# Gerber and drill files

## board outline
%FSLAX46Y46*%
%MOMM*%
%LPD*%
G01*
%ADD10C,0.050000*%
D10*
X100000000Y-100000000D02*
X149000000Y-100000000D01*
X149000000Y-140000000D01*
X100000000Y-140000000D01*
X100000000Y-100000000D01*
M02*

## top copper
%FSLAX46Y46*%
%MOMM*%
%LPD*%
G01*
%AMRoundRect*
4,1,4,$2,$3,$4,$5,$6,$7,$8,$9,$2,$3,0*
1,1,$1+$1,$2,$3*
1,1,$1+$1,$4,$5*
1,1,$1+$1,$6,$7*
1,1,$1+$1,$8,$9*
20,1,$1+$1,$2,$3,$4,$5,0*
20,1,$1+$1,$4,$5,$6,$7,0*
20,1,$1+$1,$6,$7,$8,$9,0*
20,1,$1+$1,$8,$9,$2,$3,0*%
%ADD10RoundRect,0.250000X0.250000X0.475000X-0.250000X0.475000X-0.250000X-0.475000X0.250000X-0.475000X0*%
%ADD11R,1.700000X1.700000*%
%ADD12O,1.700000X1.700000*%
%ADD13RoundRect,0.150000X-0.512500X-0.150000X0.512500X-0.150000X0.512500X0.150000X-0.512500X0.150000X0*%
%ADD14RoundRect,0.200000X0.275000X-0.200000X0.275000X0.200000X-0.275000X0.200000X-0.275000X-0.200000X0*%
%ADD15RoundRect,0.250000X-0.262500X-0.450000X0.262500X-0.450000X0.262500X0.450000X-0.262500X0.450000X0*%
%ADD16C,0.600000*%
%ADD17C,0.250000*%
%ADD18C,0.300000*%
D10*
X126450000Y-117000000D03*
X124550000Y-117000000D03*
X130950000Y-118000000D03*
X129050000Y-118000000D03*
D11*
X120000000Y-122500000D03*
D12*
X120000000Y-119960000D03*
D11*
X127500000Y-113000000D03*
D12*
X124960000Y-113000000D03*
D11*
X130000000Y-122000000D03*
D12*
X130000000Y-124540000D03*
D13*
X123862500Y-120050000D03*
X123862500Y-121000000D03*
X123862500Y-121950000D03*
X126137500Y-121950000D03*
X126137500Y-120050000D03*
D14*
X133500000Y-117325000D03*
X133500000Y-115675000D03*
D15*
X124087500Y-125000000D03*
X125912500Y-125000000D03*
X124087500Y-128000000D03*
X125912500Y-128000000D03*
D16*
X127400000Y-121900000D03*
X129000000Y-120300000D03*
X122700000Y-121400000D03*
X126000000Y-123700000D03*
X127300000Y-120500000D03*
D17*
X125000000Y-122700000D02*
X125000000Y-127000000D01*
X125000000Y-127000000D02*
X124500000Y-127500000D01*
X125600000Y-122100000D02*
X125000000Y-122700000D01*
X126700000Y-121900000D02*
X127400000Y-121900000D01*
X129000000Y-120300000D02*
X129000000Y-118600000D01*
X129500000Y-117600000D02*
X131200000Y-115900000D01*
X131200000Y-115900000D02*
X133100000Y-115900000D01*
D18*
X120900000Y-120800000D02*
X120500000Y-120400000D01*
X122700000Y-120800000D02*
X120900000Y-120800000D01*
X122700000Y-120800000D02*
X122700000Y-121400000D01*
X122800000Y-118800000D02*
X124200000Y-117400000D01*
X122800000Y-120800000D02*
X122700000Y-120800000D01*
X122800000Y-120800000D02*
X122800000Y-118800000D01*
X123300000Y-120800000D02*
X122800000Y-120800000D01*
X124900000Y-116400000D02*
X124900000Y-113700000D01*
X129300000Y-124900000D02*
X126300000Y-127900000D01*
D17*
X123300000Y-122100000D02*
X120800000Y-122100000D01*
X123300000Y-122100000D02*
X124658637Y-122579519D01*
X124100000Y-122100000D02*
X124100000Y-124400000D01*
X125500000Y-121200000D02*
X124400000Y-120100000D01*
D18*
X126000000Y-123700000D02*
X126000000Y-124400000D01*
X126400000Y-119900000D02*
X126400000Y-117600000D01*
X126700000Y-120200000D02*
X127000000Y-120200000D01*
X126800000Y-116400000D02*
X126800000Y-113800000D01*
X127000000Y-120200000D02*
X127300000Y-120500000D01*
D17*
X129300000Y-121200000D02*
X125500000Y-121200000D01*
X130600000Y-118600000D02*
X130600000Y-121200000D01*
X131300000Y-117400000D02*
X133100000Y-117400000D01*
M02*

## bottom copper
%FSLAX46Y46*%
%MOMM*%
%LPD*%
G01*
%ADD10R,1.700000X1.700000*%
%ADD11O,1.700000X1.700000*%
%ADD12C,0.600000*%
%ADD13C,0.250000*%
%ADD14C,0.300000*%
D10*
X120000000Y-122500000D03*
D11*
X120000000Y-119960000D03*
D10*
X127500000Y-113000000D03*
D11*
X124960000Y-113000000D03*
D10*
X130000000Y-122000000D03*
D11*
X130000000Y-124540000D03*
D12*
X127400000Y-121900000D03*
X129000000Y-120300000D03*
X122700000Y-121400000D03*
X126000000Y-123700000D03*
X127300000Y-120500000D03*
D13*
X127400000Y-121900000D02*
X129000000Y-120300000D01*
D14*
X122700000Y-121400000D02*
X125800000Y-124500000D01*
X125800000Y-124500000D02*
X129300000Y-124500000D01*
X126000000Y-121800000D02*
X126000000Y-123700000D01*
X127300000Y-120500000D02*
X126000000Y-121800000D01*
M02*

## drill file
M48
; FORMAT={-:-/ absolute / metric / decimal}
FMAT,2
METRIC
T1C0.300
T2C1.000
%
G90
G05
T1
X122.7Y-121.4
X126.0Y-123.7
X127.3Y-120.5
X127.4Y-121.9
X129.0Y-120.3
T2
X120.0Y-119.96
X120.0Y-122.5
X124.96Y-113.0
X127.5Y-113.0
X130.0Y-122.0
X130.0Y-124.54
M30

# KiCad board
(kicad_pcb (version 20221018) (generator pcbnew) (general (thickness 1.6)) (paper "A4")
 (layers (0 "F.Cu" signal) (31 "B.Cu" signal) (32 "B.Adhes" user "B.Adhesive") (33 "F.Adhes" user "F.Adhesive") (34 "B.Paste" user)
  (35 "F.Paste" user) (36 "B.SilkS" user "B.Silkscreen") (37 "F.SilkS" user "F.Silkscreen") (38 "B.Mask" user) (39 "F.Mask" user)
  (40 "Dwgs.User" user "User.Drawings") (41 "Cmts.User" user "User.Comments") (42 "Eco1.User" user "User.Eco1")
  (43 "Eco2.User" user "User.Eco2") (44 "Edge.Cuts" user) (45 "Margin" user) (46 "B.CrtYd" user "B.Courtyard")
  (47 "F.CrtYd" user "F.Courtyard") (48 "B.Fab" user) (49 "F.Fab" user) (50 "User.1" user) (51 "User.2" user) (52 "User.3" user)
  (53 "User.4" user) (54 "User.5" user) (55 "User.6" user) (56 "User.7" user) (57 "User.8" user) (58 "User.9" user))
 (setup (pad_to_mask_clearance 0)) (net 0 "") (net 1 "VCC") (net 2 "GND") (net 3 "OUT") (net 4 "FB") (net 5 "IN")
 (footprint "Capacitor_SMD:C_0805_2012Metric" (layer "F.Cu") (at 125.5 117 180)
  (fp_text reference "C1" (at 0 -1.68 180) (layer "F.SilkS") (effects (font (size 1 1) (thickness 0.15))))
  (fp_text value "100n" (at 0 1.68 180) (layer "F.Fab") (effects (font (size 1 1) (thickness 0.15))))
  (pad "1" smd roundrect (at -0.95 0 180) (size 1 1.45) (layers "F.Cu" "F.Paste" "F.Mask") (roundrect_rratio 0.25) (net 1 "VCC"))
  (pad "2" smd roundrect (at 0.95 0 180) (size 1 1.45) (layers "F.Cu" "F.Paste" "F.Mask") (roundrect_rratio 0.25) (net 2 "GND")))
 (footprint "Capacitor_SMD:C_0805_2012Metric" (layer "F.Cu") (at 130 118 180)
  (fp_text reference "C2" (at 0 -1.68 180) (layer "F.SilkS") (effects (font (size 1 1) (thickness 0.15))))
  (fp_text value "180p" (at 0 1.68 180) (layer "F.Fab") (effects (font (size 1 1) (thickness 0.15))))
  (pad "1" smd roundrect (at -0.95 0 180) (size 1 1.45) (layers "F.Cu" "F.Paste" "F.Mask") (roundrect_rratio 0.25) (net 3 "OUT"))
  (pad "2" smd roundrect (at 0.95 0 180) (size 1 1.45) (layers "F.Cu" "F.Paste" "F.Mask") (roundrect_rratio 0.25) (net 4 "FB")))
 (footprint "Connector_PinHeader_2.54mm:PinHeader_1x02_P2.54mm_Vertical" (layer "F.Cu") (at 120 122.5 180)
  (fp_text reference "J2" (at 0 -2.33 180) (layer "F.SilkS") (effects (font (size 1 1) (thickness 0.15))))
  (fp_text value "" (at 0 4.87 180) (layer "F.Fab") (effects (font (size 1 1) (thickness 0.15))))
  (pad "1" thru_hole rect (at 0 0 180) (size 1.7 1.7) (drill 1) (layers "*.Cu" "*.Mask") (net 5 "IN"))
  (pad "2" thru_hole oval (at 0 2.54 180) (size 1.7 1.7) (drill 1) (layers "*.Cu" "*.Mask") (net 2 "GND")))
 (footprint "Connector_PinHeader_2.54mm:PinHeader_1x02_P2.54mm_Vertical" (layer "F.Cu") (at 127.5 113 -90)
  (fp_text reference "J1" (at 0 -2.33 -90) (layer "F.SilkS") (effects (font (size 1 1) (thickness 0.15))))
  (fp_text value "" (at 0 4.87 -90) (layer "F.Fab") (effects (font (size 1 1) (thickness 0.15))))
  (pad "1" thru_hole rect (at 0 0 270) (size 1.7 1.7) (drill 1) (layers "*.Cu" "*.Mask") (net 1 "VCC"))
  (pad "2" thru_hole oval (at 0 2.54 270) (size 1.7 1.7) (drill 1) (layers "*.Cu" "*.Mask") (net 2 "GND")))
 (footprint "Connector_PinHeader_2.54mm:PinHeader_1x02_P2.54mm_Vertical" (layer "F.Cu") (at 130 122)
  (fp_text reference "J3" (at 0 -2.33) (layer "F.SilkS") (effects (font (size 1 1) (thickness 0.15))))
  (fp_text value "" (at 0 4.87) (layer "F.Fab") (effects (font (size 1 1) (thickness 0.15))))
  (pad "1" thru_hole rect (at 0 0) (size 1.7 1.7) (drill 1) (layers "*.Cu" "*.Mask") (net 3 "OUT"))
  (pad "2" thru_hole oval (at 0 2.54) (size 1.7 1.7) (drill 1) (layers "*.Cu" "*.Mask") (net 2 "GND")))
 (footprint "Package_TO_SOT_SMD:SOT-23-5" (layer "F.Cu") (at 125 121)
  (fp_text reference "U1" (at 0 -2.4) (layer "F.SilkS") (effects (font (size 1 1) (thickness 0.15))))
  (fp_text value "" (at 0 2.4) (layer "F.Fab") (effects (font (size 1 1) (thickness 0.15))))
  (pad "1" smd roundrect (at -1.1375 -0.95) (size 1.325 0.6) (layers "F.Cu" "F.Paste" "F.Mask") (roundrect_rratio 0.25) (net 3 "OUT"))
  (pad "2" smd roundrect (at -1.1375 0) (size 1.325 0.6) (layers "F.Cu" "F.Paste" "F.Mask") (roundrect_rratio 0.25) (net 2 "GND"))
  (pad "3" smd roundrect (at -1.1375 0.95) (size 1.325 0.6) (layers "F.Cu" "F.Paste" "F.Mask") (roundrect_rratio 0.25) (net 5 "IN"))
  (pad "4" smd roundrect (at 1.1375 0.95) (size 1.325 0.6) (layers "F.Cu" "F.Paste" "F.Mask") (roundrect_rratio 0.25) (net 4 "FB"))
  (pad "5" smd roundrect (at 1.1375 -0.95) (size 1.325 0.6) (layers "F.Cu" "F.Paste" "F.Mask") (roundrect_rratio 0.25) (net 1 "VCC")))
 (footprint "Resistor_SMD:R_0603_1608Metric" (layer "F.Cu") (at 133.5 116.5 90)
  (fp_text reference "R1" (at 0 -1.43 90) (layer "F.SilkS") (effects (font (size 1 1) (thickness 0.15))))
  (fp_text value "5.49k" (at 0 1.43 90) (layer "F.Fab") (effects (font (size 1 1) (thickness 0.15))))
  (pad "1" smd roundrect (at -0.825 0 90) (size 0.8 0.95) (layers "F.Cu" "F.Paste" "F.Mask") (roundrect_rratio 0.25) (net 3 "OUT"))
  (pad "2" smd roundrect (at 0.825 0 90) (size 0.8 0.95) (layers "F.Cu" "F.Paste" "F.Mask") (roundrect_rratio 0.25) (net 4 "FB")))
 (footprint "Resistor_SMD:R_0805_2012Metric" (layer "F.Cu") (at 125 125)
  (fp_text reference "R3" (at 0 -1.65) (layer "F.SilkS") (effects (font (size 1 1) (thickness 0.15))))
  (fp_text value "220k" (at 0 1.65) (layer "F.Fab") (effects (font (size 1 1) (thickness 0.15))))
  (pad "1" smd roundrect (at -0.9125 0) (size 1.025 1.4) (layers "F.Cu" "F.Paste" "F.Mask") (roundrect_rratio 0.243902) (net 5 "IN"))
  (pad "2" smd roundrect (at 0.9125 0) (size 1.025 1.4) (layers "F.Cu" "F.Paste" "F.Mask") (roundrect_rratio 0.243902) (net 1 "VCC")))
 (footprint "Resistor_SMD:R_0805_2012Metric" (layer "F.Cu") (at 125 128)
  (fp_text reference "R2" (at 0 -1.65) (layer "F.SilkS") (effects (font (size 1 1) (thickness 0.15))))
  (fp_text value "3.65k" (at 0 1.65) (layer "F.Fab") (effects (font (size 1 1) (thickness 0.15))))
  (pad "1" smd roundrect (at -0.9125 0) (size 1.025 1.4) (layers "F.Cu" "F.Paste" "F.Mask") (roundrect_rratio 0.243902) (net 4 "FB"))
  (pad "2" smd roundrect (at 0.9125 0) (size 1.025 1.4) (layers "F.Cu" "F.Paste" "F.Mask") (roundrect_rratio 0.243902) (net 2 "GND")))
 (gr_rect (start 100 100) (end 149 140) (stroke (width 0.05) (type default)) (fill none) (layer "Edge.Cuts"))
 (segment (start 125 122.7) (end 125 127) (width 0.25) (layer "F.Cu") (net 4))
 (segment (start 125 127) (end 124.5 127.5) (width 0.25) (layer "F.Cu") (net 4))
 (segment (start 125.6 122.1) (end 125 122.7) (width 0.25) (layer "F.Cu") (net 4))
 (segment (start 126.7 121.9) (end 127.4 121.9) (width 0.25) (layer "F.Cu") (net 4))
 (segment (start 129 120.3) (end 129 118.6) (width 0.25) (layer "F.Cu") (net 4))
 (segment (start 129.5 117.6) (end 131.2 115.9) (width 0.25) (layer "F.Cu") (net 4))
 (segment (start 131.2 115.9) (end 133.1 115.9) (width 0.25) (layer "F.Cu") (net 4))
 (via (at 127.4 121.9) (size 0.6) (drill 0.3) (layers "F.Cu" "B.Cu") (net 4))
 (via (at 129 120.3) (size 0.6) (drill 0.3) (layers "F.Cu" "B.Cu") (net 4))
 (segment (start 120.9 120.8) (end 120.5 120.4) (width 0.3) (layer "F.Cu") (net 2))
 (segment (start 122.7 120.8) (end 120.9 120.8) (width 0.3) (layer "F.Cu") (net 2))
 (segment (start 122.7 120.8) (end 122.7 121.4) (width 0.3) (layer "F.Cu") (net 2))
 (segment (start 122.8 118.8) (end 124.2 117.4) (width 0.3) (layer "F.Cu") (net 2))
 (segment (start 122.8 120.8) (end 122.7 120.8) (width 0.3) (layer "F.Cu") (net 2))
 (segment (start 122.8 120.8) (end 122.8 118.8) (width 0.3) (layer "F.Cu") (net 2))
 (segment (start 123.3 120.8) (end 122.8 120.8) (width 0.3) (layer "F.Cu") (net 2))
 (segment (start 124.9 116.4) (end 124.9 113.7) (width 0.3) (layer "F.Cu") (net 2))
 (segment (start 127.4 121.9) (end 129 120.3) (width 0.25) (layer "B.Cu") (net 4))
 (segment (start 129.3 124.9) (end 126.3 127.9) (width 0.3) (layer "F.Cu") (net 2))
 (via (at 122.7 121.4) (size 0.6) (drill 0.3) (layers "F.Cu" "B.Cu") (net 2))
 (segment (start 122.7 121.4) (end 125.8 124.5) (width 0.3) (layer "B.Cu") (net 2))
 (segment (start 123.3 122.1) (end 120.8 122.1) (width 0.25) (layer "F.Cu") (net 5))
 (segment (start 123.3 122.1) (end 124.658637 122.579519) (width 0.25) (layer "F.Cu") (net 5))
 (segment (start 124.1 122.1) (end 124.1 124.4) (width 0.25) (layer "F.Cu") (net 5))
 (segment (start 125.5 121.2) (end 124.4 120.1) (width 0.25) (layer "F.Cu") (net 3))
 (segment (start 125.8 124.5) (end 129.3 124.5) (width 0.3) (layer "B.Cu") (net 2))
 (segment (start 126 123.7) (end 126 124.4) (width 0.3) (layer "F.Cu") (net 1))
 (segment (start 126.4 119.9) (end 126.4 117.6) (width 0.3) (layer "F.Cu") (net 1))
 (segment (start 126.7 120.2) (end 127 120.2) (width 0.3) (layer "F.Cu") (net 1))
 (segment (start 126.8 116.4) (end 126.8 113.8) (width 0.3) (layer "F.Cu") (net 1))
 (segment (start 127 120.2) (end 127.3 120.5) (width 0.3) (layer "F.Cu") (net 1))
 (segment (start 129.3 121.2) (end 125.5 121.2) (width 0.25) (layer "F.Cu") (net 3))
 (segment (start 130.6 118.6) (end 130.6 121.2) (width 0.25) (layer "F.Cu") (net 3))
 (segment (start 131.3 117.4) (end 133.1 117.4) (width 0.25) (layer "F.Cu") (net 3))
 (via (at 126 123.7) (size 0.6) (drill 0.3) (layers "F.Cu" "B.Cu") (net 1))
 (via (at 127.3 120.5) (size 0.6) (drill 0.3) (layers "F.Cu" "B.Cu") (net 1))
 (segment (start 126 121.8) (end 126 123.7) (width 0.3) (layer "B.Cu") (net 1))
 (segment (start 127.3 120.5) (end 126 121.8) (width 0.3) (layer "B.Cu") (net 1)))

